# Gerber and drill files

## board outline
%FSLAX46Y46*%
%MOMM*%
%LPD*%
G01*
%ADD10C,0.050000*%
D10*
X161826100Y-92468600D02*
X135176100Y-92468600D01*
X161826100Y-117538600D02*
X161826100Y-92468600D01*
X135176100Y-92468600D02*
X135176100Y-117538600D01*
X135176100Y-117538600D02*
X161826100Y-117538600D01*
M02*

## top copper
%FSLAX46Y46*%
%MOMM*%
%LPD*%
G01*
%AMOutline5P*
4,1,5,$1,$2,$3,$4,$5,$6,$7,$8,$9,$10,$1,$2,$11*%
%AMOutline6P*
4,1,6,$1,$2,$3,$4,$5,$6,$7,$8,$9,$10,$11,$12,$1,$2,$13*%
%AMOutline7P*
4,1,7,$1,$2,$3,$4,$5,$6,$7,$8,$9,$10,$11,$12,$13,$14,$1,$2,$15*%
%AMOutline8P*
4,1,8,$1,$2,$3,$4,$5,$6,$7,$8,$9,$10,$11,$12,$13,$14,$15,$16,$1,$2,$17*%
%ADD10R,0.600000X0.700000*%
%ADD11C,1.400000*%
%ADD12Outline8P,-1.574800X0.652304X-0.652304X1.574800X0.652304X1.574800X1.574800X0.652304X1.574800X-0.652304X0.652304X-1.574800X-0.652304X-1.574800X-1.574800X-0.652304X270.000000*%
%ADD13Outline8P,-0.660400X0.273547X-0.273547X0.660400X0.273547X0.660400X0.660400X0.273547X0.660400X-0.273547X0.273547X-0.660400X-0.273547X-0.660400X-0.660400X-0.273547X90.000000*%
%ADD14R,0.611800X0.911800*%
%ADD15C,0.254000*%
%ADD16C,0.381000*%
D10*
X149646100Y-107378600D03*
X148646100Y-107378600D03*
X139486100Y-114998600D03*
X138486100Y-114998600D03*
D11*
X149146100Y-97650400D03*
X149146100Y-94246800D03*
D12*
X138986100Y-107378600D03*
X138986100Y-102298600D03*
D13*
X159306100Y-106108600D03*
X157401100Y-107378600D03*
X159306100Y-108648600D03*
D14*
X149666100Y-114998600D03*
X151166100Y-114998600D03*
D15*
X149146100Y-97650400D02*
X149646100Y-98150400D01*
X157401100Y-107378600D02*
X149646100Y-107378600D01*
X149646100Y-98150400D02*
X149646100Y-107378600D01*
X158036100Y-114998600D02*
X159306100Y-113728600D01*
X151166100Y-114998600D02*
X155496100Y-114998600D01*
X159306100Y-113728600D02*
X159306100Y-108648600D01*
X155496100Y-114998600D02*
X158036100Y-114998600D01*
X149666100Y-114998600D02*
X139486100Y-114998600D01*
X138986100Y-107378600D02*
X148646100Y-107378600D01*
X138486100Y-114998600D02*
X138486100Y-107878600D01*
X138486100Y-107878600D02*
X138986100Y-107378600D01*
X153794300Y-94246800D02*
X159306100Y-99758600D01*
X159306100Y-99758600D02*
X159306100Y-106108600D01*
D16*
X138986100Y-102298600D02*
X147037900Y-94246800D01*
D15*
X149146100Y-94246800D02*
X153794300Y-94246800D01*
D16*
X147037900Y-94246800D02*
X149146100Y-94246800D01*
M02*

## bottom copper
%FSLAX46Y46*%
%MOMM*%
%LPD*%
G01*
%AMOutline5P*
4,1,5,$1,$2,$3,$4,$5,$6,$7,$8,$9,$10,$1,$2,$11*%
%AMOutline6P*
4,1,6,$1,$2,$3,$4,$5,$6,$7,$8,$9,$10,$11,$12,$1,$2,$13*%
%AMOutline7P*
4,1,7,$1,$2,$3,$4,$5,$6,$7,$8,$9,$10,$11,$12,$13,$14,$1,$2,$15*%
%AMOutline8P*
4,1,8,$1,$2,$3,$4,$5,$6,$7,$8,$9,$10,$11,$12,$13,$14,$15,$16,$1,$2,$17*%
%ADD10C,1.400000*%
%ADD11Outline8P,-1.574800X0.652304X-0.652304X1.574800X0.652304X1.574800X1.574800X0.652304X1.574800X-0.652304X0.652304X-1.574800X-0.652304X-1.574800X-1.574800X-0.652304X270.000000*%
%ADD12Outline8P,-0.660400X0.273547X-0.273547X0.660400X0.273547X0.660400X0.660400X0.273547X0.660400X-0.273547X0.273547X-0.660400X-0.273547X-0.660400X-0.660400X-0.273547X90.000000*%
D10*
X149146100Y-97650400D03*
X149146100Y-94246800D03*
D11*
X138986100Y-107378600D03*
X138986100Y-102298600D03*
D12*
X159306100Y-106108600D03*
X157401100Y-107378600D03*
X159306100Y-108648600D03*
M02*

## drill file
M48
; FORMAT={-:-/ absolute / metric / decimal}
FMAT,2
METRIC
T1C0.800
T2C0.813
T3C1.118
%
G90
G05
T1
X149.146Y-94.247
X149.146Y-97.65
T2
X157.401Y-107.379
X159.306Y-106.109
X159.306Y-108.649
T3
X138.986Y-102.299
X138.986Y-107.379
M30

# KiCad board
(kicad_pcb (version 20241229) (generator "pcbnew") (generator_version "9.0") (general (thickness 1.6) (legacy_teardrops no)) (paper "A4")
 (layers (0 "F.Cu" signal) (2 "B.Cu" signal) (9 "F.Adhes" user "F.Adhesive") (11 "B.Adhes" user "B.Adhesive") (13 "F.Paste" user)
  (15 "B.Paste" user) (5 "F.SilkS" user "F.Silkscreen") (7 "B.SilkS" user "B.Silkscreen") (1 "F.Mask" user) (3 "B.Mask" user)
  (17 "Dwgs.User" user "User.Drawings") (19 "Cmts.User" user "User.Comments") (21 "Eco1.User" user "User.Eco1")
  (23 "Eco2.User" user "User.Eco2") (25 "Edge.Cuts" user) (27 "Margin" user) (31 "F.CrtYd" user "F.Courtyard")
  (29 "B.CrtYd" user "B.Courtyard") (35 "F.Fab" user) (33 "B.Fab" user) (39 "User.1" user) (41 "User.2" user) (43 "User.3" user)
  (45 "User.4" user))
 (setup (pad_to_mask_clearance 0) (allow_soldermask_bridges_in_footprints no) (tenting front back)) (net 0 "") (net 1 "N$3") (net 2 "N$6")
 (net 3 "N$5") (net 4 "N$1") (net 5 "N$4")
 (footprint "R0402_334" (layer "F.Cu") (at 149.1461 107.3786 180)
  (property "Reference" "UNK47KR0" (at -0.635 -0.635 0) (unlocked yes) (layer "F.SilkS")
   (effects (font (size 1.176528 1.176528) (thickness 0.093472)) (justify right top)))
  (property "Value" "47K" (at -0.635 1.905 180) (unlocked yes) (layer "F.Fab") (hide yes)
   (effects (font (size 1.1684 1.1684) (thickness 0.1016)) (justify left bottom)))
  (pad "1" smd rect (at -0.5 0 180) (size 0.6 0.7) (layers "F.Cu" "F.Mask" "F.Paste") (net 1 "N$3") (solder_mask_margin 0.1016)
   (solder_paste_margin 0) (thermal_bridge_angle 0))
  (pad "2" smd rect (at 0.5 0 180) (size 0.6 0.7) (layers "F.Cu" "F.Mask" "F.Paste") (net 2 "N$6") (solder_mask_margin 0.1016)
   (solder_paste_margin 0) (thermal_bridge_angle 0)))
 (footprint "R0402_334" (layer "F.Cu") (at 138.9861 114.9986 180)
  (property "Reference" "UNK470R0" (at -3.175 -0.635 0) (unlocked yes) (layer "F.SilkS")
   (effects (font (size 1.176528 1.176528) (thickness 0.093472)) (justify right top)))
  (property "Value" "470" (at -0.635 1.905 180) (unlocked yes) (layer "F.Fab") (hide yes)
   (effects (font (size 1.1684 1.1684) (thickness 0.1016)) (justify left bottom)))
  (pad "1" smd rect (at -0.5 0 180) (size 0.6 0.7) (layers "F.Cu" "F.Mask" "F.Paste") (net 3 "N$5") (solder_mask_margin 0.1016)
   (solder_paste_margin 0) (thermal_bridge_angle 0))
  (pad "2" smd rect (at 0.5 0 180) (size 0.6 0.7) (layers "F.Cu" "F.Mask" "F.Paste") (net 2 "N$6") (solder_mask_margin 0.1016)
   (solder_paste_margin 0) (thermal_bridge_angle 0)))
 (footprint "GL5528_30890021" (layer "F.Cu") (at 149.1461 95.9486 90)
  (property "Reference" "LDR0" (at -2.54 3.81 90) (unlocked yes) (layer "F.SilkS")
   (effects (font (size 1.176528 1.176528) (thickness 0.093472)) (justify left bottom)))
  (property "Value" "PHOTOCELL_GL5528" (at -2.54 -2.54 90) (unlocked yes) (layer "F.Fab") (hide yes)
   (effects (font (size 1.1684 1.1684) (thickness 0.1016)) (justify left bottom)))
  (pad "1" thru_hole circle (at -1.7018 0 90) (size 1.4 1.4) (drill 0.8) (layers "*.Cu" "*.Mask") (remove_unused_layers no) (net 1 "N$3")
   (solder_mask_margin 0.1016) (thermal_bridge_angle 0))
  (pad "2" thru_hole circle (at 1.7018 0 90) (size 1.4 1.4) (drill 0.8) (layers "*.Cu" "*.Mask") (remove_unused_layers no) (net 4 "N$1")
   (solder_mask_margin 0.1016) (thermal_bridge_angle 0)))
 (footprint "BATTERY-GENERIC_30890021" (layer "F.Cu") (at 138.9861 104.8386 -90)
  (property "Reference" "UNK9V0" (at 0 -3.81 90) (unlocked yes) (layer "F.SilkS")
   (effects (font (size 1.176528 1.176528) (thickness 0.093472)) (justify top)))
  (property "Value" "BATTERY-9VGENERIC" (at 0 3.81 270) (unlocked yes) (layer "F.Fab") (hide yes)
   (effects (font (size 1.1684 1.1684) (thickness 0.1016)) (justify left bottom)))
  (pad "+" thru_hole roundrect (at 2.54 0 270) (size 3.1496 3.1496) (drill 1.1176) (layers "*.Cu" "*.Mask") (remove_unused_layers no)
   (roundrect_rratio 0.25) (chamfer_ratio 0.2928932188) (chamfer top_left top_right bottom_left bottom_right) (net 2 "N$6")
   (solder_mask_margin 0.1016) (thermal_bridge_angle 0))
  (pad "-" thru_hole roundrect (at -2.54 0 270) (size 3.1496 3.1496) (drill 1.1176) (layers "*.Cu" "*.Mask") (remove_unused_layers no)
   (roundrect_rratio 0.25) (chamfer_ratio 0.2928932188) (chamfer top_left top_right bottom_left bottom_right) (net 4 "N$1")
   (solder_mask_margin 0.1016) (thermal_bridge_angle 0)))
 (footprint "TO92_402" (layer "F.Cu") (at 159.3061 107.3786 90)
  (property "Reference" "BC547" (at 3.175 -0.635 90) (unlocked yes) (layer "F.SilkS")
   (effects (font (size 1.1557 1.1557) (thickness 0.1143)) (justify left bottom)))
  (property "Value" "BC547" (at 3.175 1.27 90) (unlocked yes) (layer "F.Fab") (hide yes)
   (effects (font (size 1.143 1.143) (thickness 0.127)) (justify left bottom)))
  (pad "1" thru_hole roundrect (at 1.27 0 90) (size 1.3208 1.3208) (drill 0.8128) (layers "*.Cu" "*.Mask") (remove_unused_layers no)
   (roundrect_rratio 0.25) (chamfer_ratio 0.2928932188) (chamfer top_left top_right bottom_left bottom_right) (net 4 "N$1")
   (solder_mask_margin 0.1016) (thermal_bridge_angle 0))
  (pad "2" thru_hole roundrect (at 0 -1.905 90) (size 1.3208 1.3208) (drill 0.8128) (layers "*.Cu" "*.Mask") (remove_unused_layers no)
   (roundrect_rratio 0.25) (chamfer_ratio 0.2928932188) (chamfer top_left top_right bottom_left bottom_right) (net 1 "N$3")
   (solder_mask_margin 0.1016) (thermal_bridge_angle 0))
  (pad "3" thru_hole roundrect (at -1.27 0 90) (size 1.3208 1.3208) (drill 0.8128) (layers "*.Cu" "*.Mask") (remove_unused_layers no)
   (roundrect_rratio 0.25) (chamfer_ratio 0.2928932188) (chamfer top_left top_right bottom_left bottom_right) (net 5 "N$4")
   (solder_mask_margin 0.1016) (thermal_bridge_angle 0)))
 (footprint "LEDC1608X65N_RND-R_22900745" (layer "F.Cu") (at 150.4161 114.9986 180)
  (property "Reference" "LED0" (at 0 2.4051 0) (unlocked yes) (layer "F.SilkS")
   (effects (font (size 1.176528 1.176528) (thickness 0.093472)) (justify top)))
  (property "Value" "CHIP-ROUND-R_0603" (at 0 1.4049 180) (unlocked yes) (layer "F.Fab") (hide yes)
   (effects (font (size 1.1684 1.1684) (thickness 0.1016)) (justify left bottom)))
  (pad "A" smd rect (at 0.75 0 180) (size 0.6118 0.9118) (layers "F.Cu" "F.Mask" "F.Paste") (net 3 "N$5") (solder_mask_margin 0.1016)
   (solder_paste_margin 0) (thermal_bridge_angle 0))
  (pad "C" smd rect (at -0.75 0 180) (size 0.6118 0.9118) (layers "F.Cu" "F.Mask" "F.Paste") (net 5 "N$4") (solder_mask_margin 0.1016)
   (solder_paste_margin 0) (thermal_bridge_angle 0)))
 (gr_line (start 161.8261 92.4686) (end 135.1761 92.4686) (stroke (width 0.05) (type solid)) (layer "Edge.Cuts"))
 (gr_line (start 161.8261 117.5386) (end 161.8261 92.4686) (stroke (width 0.05) (type solid)) (layer "Edge.Cuts"))
 (gr_line (start 135.1761 92.4686) (end 135.1761 117.5386) (stroke (width 0.05) (type solid)) (layer "Edge.Cuts"))
 (gr_line (start 135.1761 117.5386) (end 161.8261 117.5386) (stroke (width 0.05) (type solid)) (layer "Edge.Cuts"))
 (segment (start 149.1461 97.6504) (end 149.6461 98.1504) (width 0.254) (layer "F.Cu") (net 1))
 (segment (start 157.4011 107.3786) (end 149.6461 107.3786) (width 0.254) (layer "F.Cu") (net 1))
 (segment (start 149.6461 98.1504) (end 149.6461 107.3786) (width 0.254) (layer "F.Cu") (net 1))
 (segment (start 158.0361 114.9986) (end 159.3061 113.7286) (width 0.254) (layer "F.Cu") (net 5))
 (segment (start 151.1661 114.9986) (end 155.4961 114.9986) (width 0.254) (layer "F.Cu") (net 5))
 (segment (start 159.3061 113.7286) (end 159.3061 108.6486) (width 0.254) (layer "F.Cu") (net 5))
 (segment (start 155.4961 114.9986) (end 158.0361 114.9986) (width 0.254) (layer "F.Cu") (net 5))
 (segment (start 149.6661 114.9986) (end 139.4861 114.9986) (width 0.254) (layer "F.Cu") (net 3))
 (segment (start 138.9861 107.3786) (end 148.6461 107.3786) (width 0.254) (layer "F.Cu") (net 2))
 (segment (start 138.4861 114.9986) (end 138.4861 107.8786) (width 0.254) (layer "F.Cu") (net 2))
 (segment (start 138.4861 107.8786) (end 138.9861 107.3786) (width 0.254) (layer "F.Cu") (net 2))
 (segment (start 153.7943 94.2468) (end 159.3061 99.7586) (width 0.254) (layer "F.Cu") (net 4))
 (segment (start 159.3061 99.7586) (end 159.3061 106.1086) (width 0.254) (layer "F.Cu") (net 4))
 (segment (start 138.9861 102.2986) (end 147.0379 94.2468) (width 0.381) (layer "F.Cu") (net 4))
 (segment (start 149.1461 94.2468) (end 153.7943 94.2468) (width 0.254) (layer "F.Cu") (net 4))
 (segment (start 147.0379 94.2468) (end 149.1461 94.2468) (width 0.381) (layer "F.Cu") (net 4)))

